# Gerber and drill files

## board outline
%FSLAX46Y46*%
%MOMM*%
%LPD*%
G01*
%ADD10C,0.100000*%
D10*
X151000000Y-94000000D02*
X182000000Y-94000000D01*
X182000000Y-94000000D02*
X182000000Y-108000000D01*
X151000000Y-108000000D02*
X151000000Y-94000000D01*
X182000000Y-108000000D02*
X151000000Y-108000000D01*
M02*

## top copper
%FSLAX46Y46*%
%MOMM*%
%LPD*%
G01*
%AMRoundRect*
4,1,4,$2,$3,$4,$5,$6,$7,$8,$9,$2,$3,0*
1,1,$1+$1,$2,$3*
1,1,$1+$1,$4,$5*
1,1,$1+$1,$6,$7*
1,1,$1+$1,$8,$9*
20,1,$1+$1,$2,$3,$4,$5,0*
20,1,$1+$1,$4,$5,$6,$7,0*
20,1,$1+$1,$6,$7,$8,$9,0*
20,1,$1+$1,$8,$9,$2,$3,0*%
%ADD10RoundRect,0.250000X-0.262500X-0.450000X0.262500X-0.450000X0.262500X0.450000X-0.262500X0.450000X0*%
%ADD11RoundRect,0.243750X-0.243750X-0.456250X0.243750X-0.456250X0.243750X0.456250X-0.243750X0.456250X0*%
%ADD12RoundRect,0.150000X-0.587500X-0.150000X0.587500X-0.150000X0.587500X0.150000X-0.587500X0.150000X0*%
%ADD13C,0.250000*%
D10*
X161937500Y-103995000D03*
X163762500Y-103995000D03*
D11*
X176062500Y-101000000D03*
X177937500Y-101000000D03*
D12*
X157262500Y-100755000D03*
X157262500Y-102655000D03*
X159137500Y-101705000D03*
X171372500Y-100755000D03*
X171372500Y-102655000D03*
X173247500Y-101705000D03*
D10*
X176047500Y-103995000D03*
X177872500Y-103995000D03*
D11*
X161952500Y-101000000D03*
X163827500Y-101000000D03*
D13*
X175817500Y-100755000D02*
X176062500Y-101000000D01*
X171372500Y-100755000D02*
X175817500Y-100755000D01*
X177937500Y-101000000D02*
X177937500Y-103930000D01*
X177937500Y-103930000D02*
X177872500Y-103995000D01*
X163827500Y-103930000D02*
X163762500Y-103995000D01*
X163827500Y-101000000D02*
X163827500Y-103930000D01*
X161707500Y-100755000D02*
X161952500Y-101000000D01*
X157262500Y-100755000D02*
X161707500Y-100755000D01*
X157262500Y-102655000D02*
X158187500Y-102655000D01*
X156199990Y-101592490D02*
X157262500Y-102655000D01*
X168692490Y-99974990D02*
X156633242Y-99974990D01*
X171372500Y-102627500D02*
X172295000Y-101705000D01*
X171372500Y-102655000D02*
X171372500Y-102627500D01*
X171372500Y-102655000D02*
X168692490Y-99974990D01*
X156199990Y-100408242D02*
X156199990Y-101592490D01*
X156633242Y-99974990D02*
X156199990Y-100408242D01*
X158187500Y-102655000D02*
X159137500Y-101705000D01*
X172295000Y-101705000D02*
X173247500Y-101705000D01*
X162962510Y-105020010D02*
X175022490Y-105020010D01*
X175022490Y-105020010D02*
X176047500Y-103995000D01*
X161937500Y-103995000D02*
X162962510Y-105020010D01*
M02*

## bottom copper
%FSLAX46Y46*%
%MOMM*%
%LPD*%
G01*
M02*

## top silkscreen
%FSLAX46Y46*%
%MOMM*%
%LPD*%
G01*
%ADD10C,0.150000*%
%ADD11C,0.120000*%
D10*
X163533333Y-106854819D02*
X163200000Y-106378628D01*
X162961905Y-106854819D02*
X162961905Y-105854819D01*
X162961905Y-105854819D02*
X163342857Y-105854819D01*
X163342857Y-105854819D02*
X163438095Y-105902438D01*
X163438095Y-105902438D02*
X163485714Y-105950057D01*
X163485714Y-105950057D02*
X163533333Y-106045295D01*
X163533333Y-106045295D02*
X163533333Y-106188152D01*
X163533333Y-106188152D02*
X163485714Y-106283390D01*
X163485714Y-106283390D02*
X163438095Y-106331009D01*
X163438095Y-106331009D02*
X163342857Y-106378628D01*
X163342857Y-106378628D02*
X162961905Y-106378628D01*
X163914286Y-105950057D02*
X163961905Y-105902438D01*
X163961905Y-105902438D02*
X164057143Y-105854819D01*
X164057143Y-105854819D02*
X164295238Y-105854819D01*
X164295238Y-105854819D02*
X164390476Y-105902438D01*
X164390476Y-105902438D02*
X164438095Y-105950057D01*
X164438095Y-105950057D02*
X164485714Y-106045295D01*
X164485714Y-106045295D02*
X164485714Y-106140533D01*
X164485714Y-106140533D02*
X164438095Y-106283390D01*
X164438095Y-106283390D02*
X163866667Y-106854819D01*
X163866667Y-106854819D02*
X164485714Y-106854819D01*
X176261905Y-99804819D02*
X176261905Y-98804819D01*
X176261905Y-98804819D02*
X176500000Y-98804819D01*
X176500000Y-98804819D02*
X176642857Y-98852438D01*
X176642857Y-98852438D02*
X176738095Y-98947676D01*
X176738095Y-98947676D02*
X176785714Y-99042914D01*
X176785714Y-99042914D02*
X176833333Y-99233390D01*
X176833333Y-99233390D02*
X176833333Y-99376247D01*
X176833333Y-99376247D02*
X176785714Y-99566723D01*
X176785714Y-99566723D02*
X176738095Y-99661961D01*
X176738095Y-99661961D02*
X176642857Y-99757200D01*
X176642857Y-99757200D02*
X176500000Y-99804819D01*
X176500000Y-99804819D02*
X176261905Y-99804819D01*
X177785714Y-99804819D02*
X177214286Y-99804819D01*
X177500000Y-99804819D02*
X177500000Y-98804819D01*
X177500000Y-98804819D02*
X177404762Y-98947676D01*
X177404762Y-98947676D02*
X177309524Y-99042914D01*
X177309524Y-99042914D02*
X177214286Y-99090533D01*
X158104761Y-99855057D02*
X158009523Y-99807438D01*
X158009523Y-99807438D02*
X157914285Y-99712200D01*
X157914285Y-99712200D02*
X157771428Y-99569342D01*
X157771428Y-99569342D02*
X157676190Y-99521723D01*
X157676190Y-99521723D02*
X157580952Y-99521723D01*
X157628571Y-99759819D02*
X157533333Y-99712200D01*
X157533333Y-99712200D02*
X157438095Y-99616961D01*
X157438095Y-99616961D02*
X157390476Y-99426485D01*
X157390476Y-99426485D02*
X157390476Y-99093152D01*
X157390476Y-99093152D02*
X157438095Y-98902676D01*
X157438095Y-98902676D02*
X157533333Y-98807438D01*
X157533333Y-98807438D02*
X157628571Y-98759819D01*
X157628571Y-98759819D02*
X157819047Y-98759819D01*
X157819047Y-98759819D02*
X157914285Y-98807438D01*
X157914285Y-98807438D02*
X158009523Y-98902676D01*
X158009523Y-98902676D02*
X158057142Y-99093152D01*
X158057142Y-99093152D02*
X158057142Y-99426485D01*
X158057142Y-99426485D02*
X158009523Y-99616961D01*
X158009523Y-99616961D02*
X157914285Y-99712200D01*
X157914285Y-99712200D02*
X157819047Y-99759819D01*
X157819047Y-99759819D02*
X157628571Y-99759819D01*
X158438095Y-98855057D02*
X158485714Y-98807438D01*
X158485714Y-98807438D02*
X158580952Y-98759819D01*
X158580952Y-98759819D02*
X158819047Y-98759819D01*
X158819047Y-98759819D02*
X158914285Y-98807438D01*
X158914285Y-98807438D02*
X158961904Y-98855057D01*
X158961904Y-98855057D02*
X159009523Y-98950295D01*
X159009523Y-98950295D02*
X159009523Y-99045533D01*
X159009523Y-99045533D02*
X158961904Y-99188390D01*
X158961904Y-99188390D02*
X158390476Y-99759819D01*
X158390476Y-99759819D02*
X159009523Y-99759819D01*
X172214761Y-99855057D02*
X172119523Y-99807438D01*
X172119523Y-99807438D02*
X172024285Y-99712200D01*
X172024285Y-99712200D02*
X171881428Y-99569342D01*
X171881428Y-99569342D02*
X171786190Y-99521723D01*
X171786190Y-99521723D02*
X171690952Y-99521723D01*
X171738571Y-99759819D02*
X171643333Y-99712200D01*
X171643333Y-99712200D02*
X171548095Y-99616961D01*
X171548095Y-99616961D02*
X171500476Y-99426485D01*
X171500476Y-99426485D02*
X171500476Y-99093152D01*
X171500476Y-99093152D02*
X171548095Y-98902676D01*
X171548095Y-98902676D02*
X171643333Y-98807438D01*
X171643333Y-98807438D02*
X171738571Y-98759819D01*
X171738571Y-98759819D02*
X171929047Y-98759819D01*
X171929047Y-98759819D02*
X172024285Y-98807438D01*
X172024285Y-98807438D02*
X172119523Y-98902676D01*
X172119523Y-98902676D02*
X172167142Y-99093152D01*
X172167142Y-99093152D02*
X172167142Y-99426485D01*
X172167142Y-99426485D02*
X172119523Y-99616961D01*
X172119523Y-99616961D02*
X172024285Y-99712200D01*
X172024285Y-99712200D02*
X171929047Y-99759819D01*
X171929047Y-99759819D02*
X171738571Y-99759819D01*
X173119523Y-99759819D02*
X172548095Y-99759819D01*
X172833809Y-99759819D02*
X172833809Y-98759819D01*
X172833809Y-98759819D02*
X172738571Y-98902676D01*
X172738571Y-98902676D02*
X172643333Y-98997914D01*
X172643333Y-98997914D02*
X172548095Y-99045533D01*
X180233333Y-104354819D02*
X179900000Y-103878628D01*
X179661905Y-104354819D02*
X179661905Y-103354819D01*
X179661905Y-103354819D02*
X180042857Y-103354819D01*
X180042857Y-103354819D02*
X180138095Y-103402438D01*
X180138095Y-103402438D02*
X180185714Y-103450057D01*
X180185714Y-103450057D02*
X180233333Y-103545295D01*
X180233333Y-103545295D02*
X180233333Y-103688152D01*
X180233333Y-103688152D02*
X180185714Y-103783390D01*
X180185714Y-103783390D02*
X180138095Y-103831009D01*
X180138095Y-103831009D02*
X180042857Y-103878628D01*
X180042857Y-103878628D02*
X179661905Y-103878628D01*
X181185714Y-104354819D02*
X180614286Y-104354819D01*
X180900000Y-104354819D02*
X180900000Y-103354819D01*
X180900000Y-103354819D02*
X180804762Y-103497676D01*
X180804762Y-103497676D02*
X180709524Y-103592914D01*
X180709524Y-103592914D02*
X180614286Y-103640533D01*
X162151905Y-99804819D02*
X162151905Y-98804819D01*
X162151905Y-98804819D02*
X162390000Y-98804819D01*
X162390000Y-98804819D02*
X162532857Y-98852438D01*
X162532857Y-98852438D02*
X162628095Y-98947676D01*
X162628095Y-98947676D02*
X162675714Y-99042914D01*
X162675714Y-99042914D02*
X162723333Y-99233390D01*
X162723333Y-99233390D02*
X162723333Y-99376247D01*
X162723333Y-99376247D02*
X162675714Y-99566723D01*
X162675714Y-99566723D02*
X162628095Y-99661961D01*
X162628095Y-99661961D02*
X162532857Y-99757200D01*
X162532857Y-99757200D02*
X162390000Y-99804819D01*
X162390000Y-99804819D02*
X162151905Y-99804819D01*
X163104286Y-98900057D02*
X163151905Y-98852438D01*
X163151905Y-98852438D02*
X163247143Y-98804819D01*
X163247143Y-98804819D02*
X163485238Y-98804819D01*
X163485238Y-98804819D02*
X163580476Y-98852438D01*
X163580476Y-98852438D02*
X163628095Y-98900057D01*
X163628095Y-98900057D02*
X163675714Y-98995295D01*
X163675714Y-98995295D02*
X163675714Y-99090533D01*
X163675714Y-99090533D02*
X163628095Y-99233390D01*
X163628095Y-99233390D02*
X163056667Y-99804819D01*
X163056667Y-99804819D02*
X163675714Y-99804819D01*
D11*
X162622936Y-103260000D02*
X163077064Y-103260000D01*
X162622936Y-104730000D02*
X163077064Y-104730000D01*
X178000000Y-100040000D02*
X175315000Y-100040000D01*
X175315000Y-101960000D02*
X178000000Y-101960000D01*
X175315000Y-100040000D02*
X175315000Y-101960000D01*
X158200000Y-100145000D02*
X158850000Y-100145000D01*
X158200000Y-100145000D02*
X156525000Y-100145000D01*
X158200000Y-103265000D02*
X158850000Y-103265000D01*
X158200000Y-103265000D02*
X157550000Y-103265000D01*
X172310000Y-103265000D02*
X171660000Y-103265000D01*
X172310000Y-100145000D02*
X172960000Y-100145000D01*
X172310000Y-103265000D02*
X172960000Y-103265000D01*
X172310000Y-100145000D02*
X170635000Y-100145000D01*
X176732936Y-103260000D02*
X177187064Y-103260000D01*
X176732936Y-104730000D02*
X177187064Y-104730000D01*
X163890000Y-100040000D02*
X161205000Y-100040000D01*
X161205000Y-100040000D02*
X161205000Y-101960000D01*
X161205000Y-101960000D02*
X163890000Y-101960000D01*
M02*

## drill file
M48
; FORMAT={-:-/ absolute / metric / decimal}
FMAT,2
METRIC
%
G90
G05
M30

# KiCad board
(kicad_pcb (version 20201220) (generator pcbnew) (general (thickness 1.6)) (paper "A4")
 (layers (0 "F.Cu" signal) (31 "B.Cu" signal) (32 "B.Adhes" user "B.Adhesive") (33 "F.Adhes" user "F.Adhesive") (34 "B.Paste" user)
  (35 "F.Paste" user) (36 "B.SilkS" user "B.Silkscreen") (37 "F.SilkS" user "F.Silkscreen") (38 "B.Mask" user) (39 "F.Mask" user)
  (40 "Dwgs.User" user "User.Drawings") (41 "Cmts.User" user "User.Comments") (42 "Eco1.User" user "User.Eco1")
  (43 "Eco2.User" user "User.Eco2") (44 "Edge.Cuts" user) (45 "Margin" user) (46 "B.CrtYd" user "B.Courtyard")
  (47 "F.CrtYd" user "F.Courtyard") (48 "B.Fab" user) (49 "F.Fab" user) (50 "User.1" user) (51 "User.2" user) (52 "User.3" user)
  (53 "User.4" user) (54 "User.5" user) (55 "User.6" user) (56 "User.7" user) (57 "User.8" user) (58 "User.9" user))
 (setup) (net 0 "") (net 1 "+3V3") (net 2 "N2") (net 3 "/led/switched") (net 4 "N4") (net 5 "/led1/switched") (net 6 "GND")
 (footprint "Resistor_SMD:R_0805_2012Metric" (layer "F.Cu") (at 162.85 103.995)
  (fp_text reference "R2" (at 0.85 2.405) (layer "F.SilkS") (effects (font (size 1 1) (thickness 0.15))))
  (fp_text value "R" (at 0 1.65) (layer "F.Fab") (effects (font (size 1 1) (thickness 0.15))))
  (fp_line (start -0.227064 -0.735) (end 0.227064 -0.735) (layer "F.SilkS") (width 0.12))
  (fp_line (start -0.227064 0.735) (end 0.227064 0.735) (layer "F.SilkS") (width 0.12))
  (pad "1" smd roundrect (at -0.9125 0) (size 1.025 1.4) (layers "F.Cu" "F.Paste" "F.Mask") (roundrect_rratio 0.243902) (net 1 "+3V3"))
  (pad "2" smd roundrect (at 0.9125 0) (size 1.025 1.4) (layers "F.Cu" "F.Paste" "F.Mask") (roundrect_rratio 0.243902) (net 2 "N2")))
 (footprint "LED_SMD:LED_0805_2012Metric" (layer "F.Cu") (at 177 101)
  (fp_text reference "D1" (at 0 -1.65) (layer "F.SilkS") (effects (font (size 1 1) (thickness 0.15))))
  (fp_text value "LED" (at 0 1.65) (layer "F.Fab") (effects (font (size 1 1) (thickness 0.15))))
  (fp_line (start 1 -0.96) (end -1.685 -0.96) (layer "F.SilkS") (width 0.12))
  (fp_line (start -1.685 0.96) (end 1 0.96) (layer "F.SilkS") (width 0.12))
  (fp_line (start -1.685 -0.96) (end -1.685 0.96) (layer "F.SilkS") (width 0.12))
  (pad "1" smd roundrect (at -0.9375 0) (size 0.975 1.4) (layers "F.Cu" "F.Paste" "F.Mask") (roundrect_rratio 0.25) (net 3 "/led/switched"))
  (pad "2" smd roundrect (at 0.9375 0) (size 0.975 1.4) (layers "F.Cu" "F.Paste" "F.Mask") (roundrect_rratio 0.25) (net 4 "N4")))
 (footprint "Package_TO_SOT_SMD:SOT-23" (layer "F.Cu") (at 158.2 101.705)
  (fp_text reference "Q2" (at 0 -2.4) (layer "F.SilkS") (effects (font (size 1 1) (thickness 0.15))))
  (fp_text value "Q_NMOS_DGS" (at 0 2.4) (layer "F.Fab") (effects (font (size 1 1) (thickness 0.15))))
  (fp_line (start 0 -1.56) (end 0.65 -1.56) (layer "F.SilkS") (width 0.12))
  (fp_line (start 0 -1.56) (end -1.675 -1.56) (layer "F.SilkS") (width 0.12))
  (fp_line (start 0 1.56) (end 0.65 1.56) (layer "F.SilkS") (width 0.12))
  (fp_line (start 0 1.56) (end -0.65 1.56) (layer "F.SilkS") (width 0.12))
  (pad "1" smd roundrect (at -0.9375 -0.95) (size 1.475 0.6) (layers "F.Cu" "F.Paste" "F.Mask") (roundrect_rratio 0.25)
   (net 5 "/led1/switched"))
  (pad "2" smd roundrect (at -0.9375 0.95) (size 1.475 0.6) (layers "F.Cu" "F.Paste" "F.Mask") (roundrect_rratio 0.25) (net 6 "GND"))
  (pad "3" smd roundrect (at 0.9375 0) (size 1.475 0.6) (layers "F.Cu" "F.Paste" "F.Mask") (roundrect_rratio 0.25) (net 6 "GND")))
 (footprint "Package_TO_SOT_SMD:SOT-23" (layer "F.Cu") (at 172.31 101.705)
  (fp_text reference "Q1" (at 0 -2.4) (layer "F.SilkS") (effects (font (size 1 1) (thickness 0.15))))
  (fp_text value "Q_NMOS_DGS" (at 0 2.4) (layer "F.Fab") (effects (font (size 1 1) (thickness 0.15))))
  (fp_line (start 0 1.56) (end -0.65 1.56) (layer "F.SilkS") (width 0.12))
  (fp_line (start 0 -1.56) (end 0.65 -1.56) (layer "F.SilkS") (width 0.12))
  (fp_line (start 0 1.56) (end 0.65 1.56) (layer "F.SilkS") (width 0.12))
  (fp_line (start 0 -1.56) (end -1.675 -1.56) (layer "F.SilkS") (width 0.12))
  (pad "1" smd roundrect (at -0.9375 -0.95) (size 1.475 0.6) (layers "F.Cu" "F.Paste" "F.Mask") (roundrect_rratio 0.25)
   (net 3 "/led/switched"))
  (pad "2" smd roundrect (at -0.9375 0.95) (size 1.475 0.6) (layers "F.Cu" "F.Paste" "F.Mask") (roundrect_rratio 0.25) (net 6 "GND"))
  (pad "3" smd roundrect (at 0.9375 0) (size 1.475 0.6) (layers "F.Cu" "F.Paste" "F.Mask") (roundrect_rratio 0.25) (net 6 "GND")))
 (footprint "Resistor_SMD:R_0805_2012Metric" (layer "F.Cu") (at 176.96 103.995)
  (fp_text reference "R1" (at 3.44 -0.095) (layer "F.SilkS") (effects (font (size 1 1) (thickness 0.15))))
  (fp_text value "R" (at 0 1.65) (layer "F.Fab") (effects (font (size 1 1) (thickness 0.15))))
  (fp_line (start -0.227064 -0.735) (end 0.227064 -0.735) (layer "F.SilkS") (width 0.12))
  (fp_line (start -0.227064 0.735) (end 0.227064 0.735) (layer "F.SilkS") (width 0.12))
  (pad "1" smd roundrect (at -0.9125 0) (size 1.025 1.4) (layers "F.Cu" "F.Paste" "F.Mask") (roundrect_rratio 0.243902) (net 1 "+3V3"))
  (pad "2" smd roundrect (at 0.9125 0) (size 1.025 1.4) (layers "F.Cu" "F.Paste" "F.Mask") (roundrect_rratio 0.243902) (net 4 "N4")))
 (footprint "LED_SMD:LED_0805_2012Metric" (layer "F.Cu") (at 162.89 101)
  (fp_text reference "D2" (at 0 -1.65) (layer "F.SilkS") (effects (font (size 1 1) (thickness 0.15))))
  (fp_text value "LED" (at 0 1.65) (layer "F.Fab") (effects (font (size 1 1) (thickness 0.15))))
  (fp_line (start 1 -0.96) (end -1.685 -0.96) (layer "F.SilkS") (width 0.12))
  (fp_line (start -1.685 -0.96) (end -1.685 0.96) (layer "F.SilkS") (width 0.12))
  (fp_line (start -1.685 0.96) (end 1 0.96) (layer "F.SilkS") (width 0.12))
  (pad "1" smd roundrect (at -0.9375 0) (size 0.975 1.4) (layers "F.Cu" "F.Paste" "F.Mask") (roundrect_rratio 0.25) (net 5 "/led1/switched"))
  (pad "2" smd roundrect (at 0.9375 0) (size 0.975 1.4) (layers "F.Cu" "F.Paste" "F.Mask") (roundrect_rratio 0.25) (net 2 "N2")))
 (gr_line (start 151 94) (end 182 94) (layer "Edge.Cuts") (width 0.1))
 (gr_line (start 182 94) (end 182 108) (layer "Edge.Cuts") (width 0.1))
 (gr_line (start 151 108) (end 151 94) (layer "Edge.Cuts") (width 0.1))
 (gr_line (start 182 108) (end 151 108) (layer "Edge.Cuts") (width 0.1))
 (segment (start 175.8175 100.755) (end 176.0625 101) (width 0.25) (layer "F.Cu") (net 3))
 (segment (start 171.3725 100.755) (end 175.8175 100.755) (width 0.25) (layer "F.Cu") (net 3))
 (segment (start 177.9375 101) (end 177.9375 103.93) (width 0.25) (layer "F.Cu") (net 4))
 (segment (start 177.9375 103.93) (end 177.8725 103.995) (width 0.25) (layer "F.Cu") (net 4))
 (segment (start 163.8275 103.93) (end 163.7625 103.995) (width 0.25) (layer "F.Cu") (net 2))
 (segment (start 163.8275 101) (end 163.8275 103.93) (width 0.25) (layer "F.Cu") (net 2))
 (segment (start 161.7075 100.755) (end 161.9525 101) (width 0.25) (layer "F.Cu") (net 5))
 (segment (start 157.2625 100.755) (end 161.7075 100.755) (width 0.25) (layer "F.Cu") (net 5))
 (segment (start 157.2625 102.655) (end 158.1875 102.655) (width 0.25) (layer "F.Cu") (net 6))
 (segment (start 156.19999 101.59249) (end 157.2625 102.655) (width 0.25) (layer "F.Cu") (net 6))
 (segment (start 168.69249 99.97499) (end 156.633242 99.97499) (width 0.25) (layer "F.Cu") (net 6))
 (segment (start 171.3725 102.6275) (end 172.295 101.705) (width 0.25) (layer "F.Cu") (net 6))
 (segment (start 171.3725 102.655) (end 171.3725 102.6275) (width 0.25) (layer "F.Cu") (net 6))
 (segment (start 171.3725 102.655) (end 168.69249 99.97499) (width 0.25) (layer "F.Cu") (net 6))
 (segment (start 156.19999 100.408242) (end 156.19999 101.59249) (width 0.25) (layer "F.Cu") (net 6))
 (segment (start 156.633242 99.97499) (end 156.19999 100.408242) (width 0.25) (layer "F.Cu") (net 6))
 (segment (start 158.1875 102.655) (end 159.1375 101.705) (width 0.25) (layer "F.Cu") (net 6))
 (segment (start 172.295 101.705) (end 173.2475 101.705) (width 0.25) (layer "F.Cu") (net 6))
 (segment (start 162.96251 105.02001) (end 175.02249 105.02001) (width 0.25) (layer "F.Cu") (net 1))
 (segment (start 175.02249 105.02001) (end 176.0475 103.995) (width 0.25) (layer "F.Cu") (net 1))
 (segment (start 161.9375 103.995) (end 162.96251 105.02001) (width 0.25) (layer "F.Cu") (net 1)))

